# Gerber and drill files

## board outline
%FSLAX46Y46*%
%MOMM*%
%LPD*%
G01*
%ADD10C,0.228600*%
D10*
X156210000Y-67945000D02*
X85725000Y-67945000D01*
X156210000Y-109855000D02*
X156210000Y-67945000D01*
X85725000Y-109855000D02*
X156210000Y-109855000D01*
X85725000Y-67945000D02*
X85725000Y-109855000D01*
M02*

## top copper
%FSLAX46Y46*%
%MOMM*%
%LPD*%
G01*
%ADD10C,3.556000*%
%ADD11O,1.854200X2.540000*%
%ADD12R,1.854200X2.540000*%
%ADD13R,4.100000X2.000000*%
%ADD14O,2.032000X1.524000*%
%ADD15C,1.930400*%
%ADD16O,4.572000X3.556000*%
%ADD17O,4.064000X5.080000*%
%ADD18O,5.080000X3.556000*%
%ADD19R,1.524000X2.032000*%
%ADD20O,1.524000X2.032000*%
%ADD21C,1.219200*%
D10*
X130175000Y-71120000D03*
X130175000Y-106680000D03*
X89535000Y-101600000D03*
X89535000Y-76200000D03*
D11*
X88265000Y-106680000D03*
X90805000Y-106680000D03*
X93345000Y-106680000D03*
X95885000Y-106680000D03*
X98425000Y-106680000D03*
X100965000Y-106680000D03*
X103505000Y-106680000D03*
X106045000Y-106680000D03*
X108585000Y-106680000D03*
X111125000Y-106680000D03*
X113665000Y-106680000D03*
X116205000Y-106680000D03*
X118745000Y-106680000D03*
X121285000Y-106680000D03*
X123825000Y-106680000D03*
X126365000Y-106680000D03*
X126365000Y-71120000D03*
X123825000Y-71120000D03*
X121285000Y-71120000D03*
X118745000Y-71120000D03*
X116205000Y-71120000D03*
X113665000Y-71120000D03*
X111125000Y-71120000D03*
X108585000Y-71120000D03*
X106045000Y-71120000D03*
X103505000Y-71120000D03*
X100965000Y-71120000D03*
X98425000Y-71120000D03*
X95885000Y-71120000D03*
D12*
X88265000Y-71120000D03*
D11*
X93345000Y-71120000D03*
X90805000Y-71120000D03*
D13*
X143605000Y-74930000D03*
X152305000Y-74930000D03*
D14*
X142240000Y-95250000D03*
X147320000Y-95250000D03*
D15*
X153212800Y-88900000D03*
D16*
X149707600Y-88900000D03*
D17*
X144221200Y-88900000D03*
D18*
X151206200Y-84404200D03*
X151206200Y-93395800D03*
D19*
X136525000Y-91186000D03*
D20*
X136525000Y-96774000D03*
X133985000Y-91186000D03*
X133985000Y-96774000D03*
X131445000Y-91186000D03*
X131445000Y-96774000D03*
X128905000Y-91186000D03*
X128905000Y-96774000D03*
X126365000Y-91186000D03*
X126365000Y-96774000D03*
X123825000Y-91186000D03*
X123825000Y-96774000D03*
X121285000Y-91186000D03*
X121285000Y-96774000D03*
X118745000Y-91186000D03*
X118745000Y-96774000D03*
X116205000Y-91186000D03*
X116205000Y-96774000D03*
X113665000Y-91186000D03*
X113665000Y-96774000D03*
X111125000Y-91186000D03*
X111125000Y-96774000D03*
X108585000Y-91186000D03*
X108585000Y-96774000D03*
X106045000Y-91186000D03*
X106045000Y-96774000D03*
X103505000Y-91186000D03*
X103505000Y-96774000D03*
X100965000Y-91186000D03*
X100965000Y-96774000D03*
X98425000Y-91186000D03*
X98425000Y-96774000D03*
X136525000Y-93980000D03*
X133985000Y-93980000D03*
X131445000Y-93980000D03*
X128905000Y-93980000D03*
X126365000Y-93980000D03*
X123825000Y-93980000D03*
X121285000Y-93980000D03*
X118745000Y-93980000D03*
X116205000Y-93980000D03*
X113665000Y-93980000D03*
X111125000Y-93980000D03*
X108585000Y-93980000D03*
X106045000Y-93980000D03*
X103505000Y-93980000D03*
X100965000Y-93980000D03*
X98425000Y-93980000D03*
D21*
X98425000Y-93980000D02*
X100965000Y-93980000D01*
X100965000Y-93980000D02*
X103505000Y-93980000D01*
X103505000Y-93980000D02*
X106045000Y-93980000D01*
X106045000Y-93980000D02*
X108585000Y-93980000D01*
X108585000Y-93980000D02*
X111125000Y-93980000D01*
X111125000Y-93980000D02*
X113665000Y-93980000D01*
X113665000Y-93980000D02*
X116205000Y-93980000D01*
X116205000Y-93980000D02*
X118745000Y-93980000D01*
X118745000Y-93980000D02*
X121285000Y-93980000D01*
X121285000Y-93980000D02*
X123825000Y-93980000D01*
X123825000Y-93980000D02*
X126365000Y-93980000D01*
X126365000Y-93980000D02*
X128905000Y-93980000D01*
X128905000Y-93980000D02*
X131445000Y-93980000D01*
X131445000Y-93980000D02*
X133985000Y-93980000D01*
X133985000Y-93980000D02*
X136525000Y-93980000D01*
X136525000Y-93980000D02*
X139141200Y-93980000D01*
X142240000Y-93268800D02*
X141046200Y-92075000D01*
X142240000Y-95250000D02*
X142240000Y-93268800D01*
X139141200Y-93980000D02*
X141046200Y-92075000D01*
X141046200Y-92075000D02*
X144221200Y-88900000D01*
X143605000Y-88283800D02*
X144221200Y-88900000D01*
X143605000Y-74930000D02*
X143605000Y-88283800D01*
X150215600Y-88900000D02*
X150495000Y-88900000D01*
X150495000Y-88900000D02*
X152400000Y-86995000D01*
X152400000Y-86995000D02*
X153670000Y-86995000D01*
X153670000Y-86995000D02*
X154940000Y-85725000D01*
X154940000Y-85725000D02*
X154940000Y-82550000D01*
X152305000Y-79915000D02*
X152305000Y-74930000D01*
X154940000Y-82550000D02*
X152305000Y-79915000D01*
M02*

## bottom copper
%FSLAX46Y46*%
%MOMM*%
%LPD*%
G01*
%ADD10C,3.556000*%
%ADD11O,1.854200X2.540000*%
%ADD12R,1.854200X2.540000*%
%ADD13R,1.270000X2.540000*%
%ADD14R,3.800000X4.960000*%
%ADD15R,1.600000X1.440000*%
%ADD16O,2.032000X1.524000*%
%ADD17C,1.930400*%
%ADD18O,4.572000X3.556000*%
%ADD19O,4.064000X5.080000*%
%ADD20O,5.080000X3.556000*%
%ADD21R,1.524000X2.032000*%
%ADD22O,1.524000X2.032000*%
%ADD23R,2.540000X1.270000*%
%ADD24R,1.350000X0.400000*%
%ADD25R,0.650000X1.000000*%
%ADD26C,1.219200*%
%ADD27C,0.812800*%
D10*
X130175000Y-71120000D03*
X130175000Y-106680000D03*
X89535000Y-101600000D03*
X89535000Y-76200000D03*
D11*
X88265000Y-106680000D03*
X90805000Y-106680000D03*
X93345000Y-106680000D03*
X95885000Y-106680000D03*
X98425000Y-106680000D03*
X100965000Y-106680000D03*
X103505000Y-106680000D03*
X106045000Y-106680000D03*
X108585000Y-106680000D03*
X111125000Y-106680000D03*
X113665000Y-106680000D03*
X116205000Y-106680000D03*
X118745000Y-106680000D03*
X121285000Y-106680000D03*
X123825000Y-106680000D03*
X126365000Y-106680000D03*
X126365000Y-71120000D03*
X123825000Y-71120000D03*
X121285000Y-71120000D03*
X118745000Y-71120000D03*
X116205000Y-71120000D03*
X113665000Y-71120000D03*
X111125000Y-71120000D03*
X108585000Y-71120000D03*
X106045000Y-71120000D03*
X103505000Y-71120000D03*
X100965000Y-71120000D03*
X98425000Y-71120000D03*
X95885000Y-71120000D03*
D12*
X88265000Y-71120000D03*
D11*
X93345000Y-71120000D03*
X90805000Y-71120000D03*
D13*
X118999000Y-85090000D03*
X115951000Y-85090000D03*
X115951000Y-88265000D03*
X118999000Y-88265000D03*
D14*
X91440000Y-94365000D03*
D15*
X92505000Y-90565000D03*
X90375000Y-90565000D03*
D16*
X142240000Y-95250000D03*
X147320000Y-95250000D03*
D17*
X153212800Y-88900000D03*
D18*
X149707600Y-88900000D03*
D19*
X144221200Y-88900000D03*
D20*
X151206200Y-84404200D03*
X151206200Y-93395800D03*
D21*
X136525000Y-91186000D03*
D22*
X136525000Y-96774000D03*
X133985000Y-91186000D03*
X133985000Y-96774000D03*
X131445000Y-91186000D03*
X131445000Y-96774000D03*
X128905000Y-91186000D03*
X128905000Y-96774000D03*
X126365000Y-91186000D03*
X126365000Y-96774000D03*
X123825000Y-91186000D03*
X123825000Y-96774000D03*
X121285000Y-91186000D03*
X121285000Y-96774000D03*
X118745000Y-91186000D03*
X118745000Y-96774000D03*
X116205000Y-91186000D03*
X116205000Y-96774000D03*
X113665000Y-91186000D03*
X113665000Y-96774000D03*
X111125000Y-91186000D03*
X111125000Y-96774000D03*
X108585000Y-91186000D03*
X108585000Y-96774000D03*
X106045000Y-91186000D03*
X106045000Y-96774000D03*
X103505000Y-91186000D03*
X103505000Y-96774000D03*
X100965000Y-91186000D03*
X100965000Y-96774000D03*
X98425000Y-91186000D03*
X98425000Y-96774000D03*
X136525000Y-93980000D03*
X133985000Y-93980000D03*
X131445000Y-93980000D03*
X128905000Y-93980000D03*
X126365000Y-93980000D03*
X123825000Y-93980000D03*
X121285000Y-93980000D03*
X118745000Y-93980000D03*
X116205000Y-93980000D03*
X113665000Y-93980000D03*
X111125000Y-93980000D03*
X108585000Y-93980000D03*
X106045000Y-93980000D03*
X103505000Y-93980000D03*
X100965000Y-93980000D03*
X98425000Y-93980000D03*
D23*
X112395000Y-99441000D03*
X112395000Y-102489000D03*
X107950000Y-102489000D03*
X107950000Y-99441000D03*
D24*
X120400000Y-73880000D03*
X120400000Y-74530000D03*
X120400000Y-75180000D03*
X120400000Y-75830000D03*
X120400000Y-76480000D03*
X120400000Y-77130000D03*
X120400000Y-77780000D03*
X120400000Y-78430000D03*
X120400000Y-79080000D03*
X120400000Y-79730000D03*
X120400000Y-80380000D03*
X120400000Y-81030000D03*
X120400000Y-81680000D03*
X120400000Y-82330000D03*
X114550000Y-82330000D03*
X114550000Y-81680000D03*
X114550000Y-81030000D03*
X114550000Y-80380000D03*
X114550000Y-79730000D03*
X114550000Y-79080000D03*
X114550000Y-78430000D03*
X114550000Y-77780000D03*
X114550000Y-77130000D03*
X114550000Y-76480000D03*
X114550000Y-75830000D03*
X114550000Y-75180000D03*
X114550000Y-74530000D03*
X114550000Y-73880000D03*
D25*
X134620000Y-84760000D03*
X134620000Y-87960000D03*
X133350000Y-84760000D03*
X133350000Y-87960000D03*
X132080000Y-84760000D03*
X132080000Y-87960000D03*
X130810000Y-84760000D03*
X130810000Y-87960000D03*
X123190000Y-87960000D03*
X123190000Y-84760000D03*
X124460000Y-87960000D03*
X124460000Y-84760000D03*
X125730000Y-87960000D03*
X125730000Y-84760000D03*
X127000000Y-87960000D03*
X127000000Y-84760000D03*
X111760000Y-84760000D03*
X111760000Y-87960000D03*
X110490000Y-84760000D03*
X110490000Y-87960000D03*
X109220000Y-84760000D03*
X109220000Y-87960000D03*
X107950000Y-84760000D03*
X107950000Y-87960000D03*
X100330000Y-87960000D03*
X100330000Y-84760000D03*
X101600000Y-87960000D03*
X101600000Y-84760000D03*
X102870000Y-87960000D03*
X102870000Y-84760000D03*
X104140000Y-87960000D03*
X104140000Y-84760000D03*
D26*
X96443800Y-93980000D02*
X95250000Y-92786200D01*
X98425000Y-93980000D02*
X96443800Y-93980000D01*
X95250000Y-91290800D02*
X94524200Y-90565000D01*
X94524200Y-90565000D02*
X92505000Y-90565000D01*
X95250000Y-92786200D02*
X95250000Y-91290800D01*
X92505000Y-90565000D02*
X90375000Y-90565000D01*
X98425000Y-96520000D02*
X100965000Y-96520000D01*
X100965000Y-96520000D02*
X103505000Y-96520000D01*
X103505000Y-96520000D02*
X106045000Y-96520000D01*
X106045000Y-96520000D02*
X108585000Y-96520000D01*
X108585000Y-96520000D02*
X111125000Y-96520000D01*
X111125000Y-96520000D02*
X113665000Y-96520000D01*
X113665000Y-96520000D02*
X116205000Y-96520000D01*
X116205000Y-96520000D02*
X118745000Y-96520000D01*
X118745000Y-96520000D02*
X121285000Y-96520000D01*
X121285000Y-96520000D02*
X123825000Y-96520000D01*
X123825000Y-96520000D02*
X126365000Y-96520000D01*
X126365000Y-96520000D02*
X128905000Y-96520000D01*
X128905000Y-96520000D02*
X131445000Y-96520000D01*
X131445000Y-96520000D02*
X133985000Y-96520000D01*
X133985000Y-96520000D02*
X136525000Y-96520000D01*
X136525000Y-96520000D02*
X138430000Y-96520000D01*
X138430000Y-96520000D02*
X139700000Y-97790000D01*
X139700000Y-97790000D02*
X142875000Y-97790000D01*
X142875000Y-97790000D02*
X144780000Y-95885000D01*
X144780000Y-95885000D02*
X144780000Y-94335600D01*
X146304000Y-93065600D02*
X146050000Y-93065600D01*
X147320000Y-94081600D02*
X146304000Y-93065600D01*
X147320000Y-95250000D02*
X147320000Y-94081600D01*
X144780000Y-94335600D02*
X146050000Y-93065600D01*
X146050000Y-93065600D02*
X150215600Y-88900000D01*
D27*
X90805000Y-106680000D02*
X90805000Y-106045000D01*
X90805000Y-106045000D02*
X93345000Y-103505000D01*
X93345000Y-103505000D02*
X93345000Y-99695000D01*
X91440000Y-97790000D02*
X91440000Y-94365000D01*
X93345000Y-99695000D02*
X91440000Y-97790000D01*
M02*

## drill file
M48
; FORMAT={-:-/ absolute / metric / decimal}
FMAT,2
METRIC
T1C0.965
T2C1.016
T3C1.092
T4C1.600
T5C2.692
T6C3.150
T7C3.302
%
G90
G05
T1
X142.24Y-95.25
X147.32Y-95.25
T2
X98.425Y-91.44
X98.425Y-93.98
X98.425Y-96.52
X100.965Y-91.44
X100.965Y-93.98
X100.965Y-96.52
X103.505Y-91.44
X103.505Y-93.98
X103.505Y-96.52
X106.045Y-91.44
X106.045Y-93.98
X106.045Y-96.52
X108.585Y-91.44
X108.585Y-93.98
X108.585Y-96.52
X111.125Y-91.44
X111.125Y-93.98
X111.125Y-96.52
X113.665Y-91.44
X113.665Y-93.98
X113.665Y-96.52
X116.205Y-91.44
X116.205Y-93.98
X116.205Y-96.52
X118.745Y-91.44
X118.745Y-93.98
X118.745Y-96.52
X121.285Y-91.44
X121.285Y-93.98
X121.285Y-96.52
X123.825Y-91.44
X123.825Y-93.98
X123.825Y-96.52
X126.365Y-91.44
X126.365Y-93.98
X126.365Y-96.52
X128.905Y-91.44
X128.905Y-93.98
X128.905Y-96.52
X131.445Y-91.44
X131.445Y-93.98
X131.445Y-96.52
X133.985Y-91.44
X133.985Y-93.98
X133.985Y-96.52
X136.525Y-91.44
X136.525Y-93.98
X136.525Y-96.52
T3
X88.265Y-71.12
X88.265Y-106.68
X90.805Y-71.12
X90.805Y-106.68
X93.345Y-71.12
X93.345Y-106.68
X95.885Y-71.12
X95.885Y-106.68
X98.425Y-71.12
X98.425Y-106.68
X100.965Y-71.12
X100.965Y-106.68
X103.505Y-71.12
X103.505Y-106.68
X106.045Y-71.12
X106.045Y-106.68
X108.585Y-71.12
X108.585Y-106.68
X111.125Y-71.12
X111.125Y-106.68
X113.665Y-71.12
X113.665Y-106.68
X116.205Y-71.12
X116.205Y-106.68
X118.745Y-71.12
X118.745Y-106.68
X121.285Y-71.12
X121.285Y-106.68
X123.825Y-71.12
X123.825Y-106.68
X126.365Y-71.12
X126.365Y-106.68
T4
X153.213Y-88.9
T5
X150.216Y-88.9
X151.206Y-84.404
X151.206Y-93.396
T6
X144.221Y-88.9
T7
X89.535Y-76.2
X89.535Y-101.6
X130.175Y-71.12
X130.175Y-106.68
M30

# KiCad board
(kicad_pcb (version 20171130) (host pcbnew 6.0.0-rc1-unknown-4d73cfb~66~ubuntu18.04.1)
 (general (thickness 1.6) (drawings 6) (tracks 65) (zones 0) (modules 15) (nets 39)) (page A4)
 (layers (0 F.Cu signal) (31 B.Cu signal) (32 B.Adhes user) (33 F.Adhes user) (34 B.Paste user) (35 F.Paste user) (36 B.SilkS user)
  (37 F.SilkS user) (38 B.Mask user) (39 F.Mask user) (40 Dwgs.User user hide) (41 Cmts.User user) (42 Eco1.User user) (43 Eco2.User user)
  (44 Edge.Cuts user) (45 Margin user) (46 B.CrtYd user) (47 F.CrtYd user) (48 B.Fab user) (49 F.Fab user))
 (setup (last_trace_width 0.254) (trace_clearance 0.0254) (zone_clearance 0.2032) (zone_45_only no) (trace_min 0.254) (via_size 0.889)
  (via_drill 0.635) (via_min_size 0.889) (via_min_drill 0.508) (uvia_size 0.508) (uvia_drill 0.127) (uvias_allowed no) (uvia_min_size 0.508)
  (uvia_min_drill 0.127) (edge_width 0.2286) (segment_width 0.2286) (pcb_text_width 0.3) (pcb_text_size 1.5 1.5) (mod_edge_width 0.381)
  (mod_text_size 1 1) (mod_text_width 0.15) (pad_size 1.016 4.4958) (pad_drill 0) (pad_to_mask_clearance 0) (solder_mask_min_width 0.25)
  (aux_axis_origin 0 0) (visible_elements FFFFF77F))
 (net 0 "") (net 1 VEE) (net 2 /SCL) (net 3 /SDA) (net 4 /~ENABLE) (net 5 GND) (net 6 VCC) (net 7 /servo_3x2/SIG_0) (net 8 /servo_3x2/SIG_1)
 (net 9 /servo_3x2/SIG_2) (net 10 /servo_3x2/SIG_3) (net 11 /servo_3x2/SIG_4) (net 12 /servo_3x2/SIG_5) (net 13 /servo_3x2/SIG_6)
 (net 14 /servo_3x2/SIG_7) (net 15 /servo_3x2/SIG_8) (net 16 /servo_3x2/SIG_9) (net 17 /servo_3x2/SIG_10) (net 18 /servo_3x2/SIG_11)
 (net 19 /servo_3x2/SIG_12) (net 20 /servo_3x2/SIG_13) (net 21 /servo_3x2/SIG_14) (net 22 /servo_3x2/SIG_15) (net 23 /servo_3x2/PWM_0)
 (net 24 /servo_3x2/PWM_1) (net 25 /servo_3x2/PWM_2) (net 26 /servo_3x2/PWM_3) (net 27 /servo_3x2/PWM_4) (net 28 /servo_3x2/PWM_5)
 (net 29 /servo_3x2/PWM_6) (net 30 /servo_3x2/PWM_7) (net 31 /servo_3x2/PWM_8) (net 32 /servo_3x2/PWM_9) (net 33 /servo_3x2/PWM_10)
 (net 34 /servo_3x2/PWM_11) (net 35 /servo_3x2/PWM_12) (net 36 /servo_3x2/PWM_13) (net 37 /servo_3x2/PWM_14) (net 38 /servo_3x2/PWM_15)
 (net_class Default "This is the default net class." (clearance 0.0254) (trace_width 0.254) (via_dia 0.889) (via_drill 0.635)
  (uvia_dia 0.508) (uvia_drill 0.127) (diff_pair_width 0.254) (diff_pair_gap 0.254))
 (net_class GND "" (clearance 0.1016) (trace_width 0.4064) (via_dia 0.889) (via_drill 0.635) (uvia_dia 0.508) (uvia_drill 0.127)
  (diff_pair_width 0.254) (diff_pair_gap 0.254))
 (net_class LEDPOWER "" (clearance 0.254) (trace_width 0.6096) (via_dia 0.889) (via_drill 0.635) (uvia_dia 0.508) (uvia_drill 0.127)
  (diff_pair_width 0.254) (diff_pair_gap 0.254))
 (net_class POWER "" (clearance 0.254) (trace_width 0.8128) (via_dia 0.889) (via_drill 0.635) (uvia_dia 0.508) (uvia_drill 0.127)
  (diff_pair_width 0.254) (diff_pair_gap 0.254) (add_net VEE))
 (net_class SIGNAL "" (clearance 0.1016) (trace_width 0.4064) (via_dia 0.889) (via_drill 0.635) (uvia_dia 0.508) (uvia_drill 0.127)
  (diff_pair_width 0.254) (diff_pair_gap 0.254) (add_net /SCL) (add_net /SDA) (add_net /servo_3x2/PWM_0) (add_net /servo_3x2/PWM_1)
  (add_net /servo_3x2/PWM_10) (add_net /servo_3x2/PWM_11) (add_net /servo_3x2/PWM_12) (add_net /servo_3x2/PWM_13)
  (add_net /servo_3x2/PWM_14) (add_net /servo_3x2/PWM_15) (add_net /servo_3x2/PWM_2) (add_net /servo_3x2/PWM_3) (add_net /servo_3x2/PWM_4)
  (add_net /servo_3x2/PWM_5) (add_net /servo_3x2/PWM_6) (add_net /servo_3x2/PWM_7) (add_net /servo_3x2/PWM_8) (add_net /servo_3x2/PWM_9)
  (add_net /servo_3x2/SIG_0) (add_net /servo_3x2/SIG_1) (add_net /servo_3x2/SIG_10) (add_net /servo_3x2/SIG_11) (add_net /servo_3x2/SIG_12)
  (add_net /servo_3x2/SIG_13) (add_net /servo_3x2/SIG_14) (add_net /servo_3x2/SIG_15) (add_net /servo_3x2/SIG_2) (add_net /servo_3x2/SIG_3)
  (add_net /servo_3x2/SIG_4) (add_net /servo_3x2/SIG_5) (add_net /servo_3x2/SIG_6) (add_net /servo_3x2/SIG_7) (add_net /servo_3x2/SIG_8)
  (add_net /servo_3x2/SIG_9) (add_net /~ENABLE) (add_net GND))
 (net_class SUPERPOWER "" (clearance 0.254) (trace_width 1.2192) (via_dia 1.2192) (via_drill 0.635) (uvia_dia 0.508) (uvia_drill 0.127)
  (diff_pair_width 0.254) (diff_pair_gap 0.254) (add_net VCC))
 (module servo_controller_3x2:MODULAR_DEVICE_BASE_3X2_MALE (layer F.Cu) (at 107.315 88.9)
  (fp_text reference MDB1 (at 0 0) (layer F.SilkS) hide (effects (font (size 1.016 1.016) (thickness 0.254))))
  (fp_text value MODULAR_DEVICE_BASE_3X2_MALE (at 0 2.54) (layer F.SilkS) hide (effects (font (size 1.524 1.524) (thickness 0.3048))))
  (pad "" thru_hole circle (at 22.86 -17.78) (size 3.556 3.556) (drill 3.302) (layers *.Cu *.Mask F.SilkS))
  (pad "" thru_hole circle (at 22.86 17.78) (size 3.556 3.556) (drill 3.302) (layers *.Cu *.Mask F.SilkS))
  (pad "" thru_hole circle (at -17.78 12.7) (size 3.556 3.556) (drill 3.302) (layers *.Cu *.Mask F.SilkS))
  (pad "" thru_hole circle (at -17.78 -12.7) (size 3.556 3.556) (drill 3.302) (layers *.Cu *.Mask F.SilkS))
  (pad AREF thru_hole oval (at -19.05 17.78) (size 1.8542 2.54) (drill 1.0922) (layers *.Cu *.Mask))
  (pad VEE thru_hole oval (at -16.51 17.78) (size 1.8542 2.54) (drill 1.0922) (layers *.Cu *.Mask) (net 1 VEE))
  (pad AGND thru_hole oval (at -13.97 17.78) (size 1.8542 2.54) (drill 1.0922) (layers *.Cu *.Mask))
  (pad 3V3 thru_hole oval (at -11.43 17.78) (size 1.8542 2.54) (drill 1.0922) (layers *.Cu *.Mask))
  (pad 23 thru_hole oval (at -8.89 17.78) (size 1.8542 2.54) (drill 1.0922) (layers *.Cu *.Mask))
  (pad 22 thru_hole oval (at -6.35 17.78) (size 1.8542 2.54) (drill 1.0922) (layers *.Cu *.Mask))
  (pad 21 thru_hole oval (at -3.81 17.78) (size 1.8542 2.54) (drill 1.0922) (layers *.Cu *.Mask))
  (pad 20 thru_hole oval (at -1.27 17.78) (size 1.8542 2.54) (drill 1.0922) (layers *.Cu *.Mask))
  (pad 19 thru_hole oval (at 1.27 17.78) (size 1.8542 2.54) (drill 1.0922) (layers *.Cu *.Mask) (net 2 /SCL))
  (pad 18 thru_hole oval (at 3.81 17.78) (size 1.8542 2.54) (drill 1.0922) (layers *.Cu *.Mask) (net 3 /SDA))
  (pad 17 thru_hole oval (at 6.35 17.78) (size 1.8542 2.54) (drill 1.0922) (layers *.Cu *.Mask))
  (pad 16 thru_hole oval (at 8.89 17.78) (size 1.8542 2.54) (drill 1.0922) (layers *.Cu *.Mask))
  (pad 15 thru_hole oval (at 11.43 17.78) (size 1.8542 2.54) (drill 1.0922) (layers *.Cu *.Mask))
  (pad 14 thru_hole oval (at 13.97 17.78) (size 1.8542 2.54) (drill 1.0922) (layers *.Cu *.Mask))
  (pad 13 thru_hole oval (at 16.51 17.78) (size 1.8542 2.54) (drill 1.0922) (layers *.Cu *.Mask))
  (pad DAC thru_hole oval (at 19.05 17.78) (size 1.8542 2.54) (drill 1.0922) (layers *.Cu *.Mask))
  (pad 28 thru_hole oval (at 19.05 -17.78) (size 1.8542 2.54) (drill 1.0922) (layers *.Cu *.Mask))
  (pad 12 thru_hole oval (at 16.51 -17.78) (size 1.8542 2.54) (drill 1.0922) (layers *.Cu *.Mask))
  (pad 11 thru_hole oval (at 13.97 -17.78) (size 1.8542 2.54) (drill 1.0922) (layers *.Cu *.Mask))
  (pad 10 thru_hole oval (at 11.43 -17.78) (size 1.8542 2.54) (drill 1.0922) (layers *.Cu *.Mask))
  (pad 9 thru_hole oval (at 8.89 -17.78) (size 1.8542 2.54) (drill 1.0922) (layers *.Cu *.Mask))
  (pad 29 thru_hole oval (at 6.35 -17.78) (size 1.8542 2.54) (drill 1.0922) (layers *.Cu *.Mask))
  (pad 30 thru_hole oval (at 3.81 -17.78) (size 1.8542 2.54) (drill 1.0922) (layers *.Cu *.Mask))
  (pad 6 thru_hole oval (at 1.27 -17.78) (size 1.8542 2.54) (drill 1.0922) (layers *.Cu *.Mask))
  (pad 5 thru_hole oval (at -1.27 -17.78) (size 1.8542 2.54) (drill 1.0922) (layers *.Cu *.Mask))
  (pad 4 thru_hole oval (at -3.81 -17.78) (size 1.8542 2.54) (drill 1.0922) (layers *.Cu *.Mask))
  (pad 3 thru_hole oval (at -6.35 -17.78) (size 1.8542 2.54) (drill 1.0922) (layers *.Cu *.Mask))
  (pad 2 thru_hole oval (at -8.89 -17.78) (size 1.8542 2.54) (drill 1.0922) (layers *.Cu *.Mask) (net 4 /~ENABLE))
  (pad 25 thru_hole oval (at -11.43 -17.78) (size 1.8542 2.54) (drill 1.0922) (layers *.Cu *.Mask))
  (pad VDD thru_hole rect (at -19.05 -17.78) (size 1.8542 2.54) (drill 1.0922) (layers *.Cu *.Mask))
  (pad 24 thru_hole oval (at -13.97 -17.78) (size 1.8542 2.54) (drill 1.0922) (layers *.Cu *.Mask))
  (pad GND thru_hole oval (at -16.51 -17.78) (size 1.8542 2.54) (drill 1.0922) (layers *.Cu *.Mask) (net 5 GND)))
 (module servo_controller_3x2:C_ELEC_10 (layer F.Cu) (at 147.955 74.93 180)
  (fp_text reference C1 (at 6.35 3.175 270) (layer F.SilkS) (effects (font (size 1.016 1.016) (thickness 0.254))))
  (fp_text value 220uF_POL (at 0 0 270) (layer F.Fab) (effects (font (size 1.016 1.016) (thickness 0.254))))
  (pad 1 smd rect (at 4.35 0 180) (size 4.1 2) (layers F.Cu F.Paste F.Mask) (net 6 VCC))
  (pad 2 smd rect (at -4.35 0 180) (size 4.1 2) (layers F.Cu F.Paste F.Mask) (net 5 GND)))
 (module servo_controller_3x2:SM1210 (layer B.Cu) (at 117.475 85.09)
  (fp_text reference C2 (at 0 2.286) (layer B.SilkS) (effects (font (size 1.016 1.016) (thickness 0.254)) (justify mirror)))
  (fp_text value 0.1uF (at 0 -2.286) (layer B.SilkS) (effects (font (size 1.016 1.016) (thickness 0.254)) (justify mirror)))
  (pad 2 smd rect (at 1.524 0) (size 1.27 2.54) (layers B.Cu B.Paste B.Mask) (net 5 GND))
  (pad 1 smd rect (at -1.524 0) (size 1.27 2.54) (layers B.Cu B.Paste B.Mask) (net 1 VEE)))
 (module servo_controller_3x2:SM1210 (layer B.Cu) (at 117.475 88.265)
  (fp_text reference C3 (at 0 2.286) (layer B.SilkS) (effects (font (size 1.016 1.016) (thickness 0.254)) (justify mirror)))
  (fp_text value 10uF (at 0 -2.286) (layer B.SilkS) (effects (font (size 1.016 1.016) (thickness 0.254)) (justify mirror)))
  (pad 1 smd rect (at -1.524 0) (size 1.27 2.54) (layers B.Cu B.Paste B.Mask) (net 1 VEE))
  (pad 2 smd rect (at 1.524 0) (size 1.27 2.54) (layers B.Cu B.Paste B.Mask) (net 5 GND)))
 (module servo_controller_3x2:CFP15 (layer B.Cu) (at 91.44 93.345 180)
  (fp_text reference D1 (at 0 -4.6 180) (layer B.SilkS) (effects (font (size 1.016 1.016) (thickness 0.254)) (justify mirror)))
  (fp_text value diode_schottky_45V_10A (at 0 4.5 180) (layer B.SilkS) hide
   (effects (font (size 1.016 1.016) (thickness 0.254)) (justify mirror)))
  (pad 1 smd rect (at 0 -1.02 180) (size 3.8 4.96) (layers B.Cu B.Paste B.Mask) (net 1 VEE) (solder_mask_margin 0.1) (clearance 0.1))
  (pad 2 smd rect (at -1.065 2.78 180) (size 1.6 1.44) (layers B.Cu B.Paste B.Mask) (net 6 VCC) (solder_mask_margin 0.1) (clearance 0.1))
  (pad 2 smd rect (at 1.065 2.78 180) (size 1.6 1.44) (layers B.Cu B.Paste B.Mask) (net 6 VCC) (solder_mask_margin 0.1) (clearance 0.1)))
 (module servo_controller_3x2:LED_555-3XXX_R (layer F.Cu) (at 144.78 95.25 90)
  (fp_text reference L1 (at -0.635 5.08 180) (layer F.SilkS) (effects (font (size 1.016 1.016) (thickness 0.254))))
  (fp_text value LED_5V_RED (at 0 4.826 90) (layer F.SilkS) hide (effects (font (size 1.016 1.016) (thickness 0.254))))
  (pad 1 thru_hole oval (at 0 -2.54 90) (size 1.524 2.032) (drill 0.9652) (layers *.Cu *.Mask) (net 6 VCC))
  (pad 2 thru_hole oval (at 0 2.54 90) (size 1.524 2.032) (drill 0.9652) (layers *.Cu *.Mask) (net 5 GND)))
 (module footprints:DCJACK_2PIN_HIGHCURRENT (layer F.Cu) (at 156.21 88.9 270)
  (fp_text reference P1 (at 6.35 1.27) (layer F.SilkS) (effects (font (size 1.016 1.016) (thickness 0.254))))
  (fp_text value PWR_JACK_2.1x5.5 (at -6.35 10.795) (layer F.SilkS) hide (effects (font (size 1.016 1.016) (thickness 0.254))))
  (pad "" thru_hole circle (at 0 2.9972 270) (size 1.9304 1.9304) (drill 1.6002) (layers *.Cu *.Mask))
  (pad 2 thru_hole oval (at 0 5.9944 270) (size 3.556 4.572) (drill 2.6924 (offset 0 0.508)) (layers *.Cu *.Mask) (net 5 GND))
  (pad 1 thru_hole oval (at 0 11.9888 270) (size 5.08 4.064) (drill 3.1496) (layers *.Cu *.Mask) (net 6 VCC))
  (pad "" thru_hole oval (at -4.4958 5.0038 270) (size 3.556 5.08) (drill 2.6924) (layers *.Cu *.Mask))
  (pad "" thru_hole oval (at 4.4958 5.0038 270) (size 3.556 5.08) (drill 2.6924) (layers *.Cu *.Mask)))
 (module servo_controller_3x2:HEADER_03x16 (layer F.Cu) (at 117.475 93.98)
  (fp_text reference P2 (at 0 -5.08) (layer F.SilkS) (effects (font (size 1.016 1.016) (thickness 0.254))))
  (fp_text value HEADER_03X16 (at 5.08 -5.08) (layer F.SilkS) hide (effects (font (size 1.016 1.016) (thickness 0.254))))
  (pad 1 thru_hole rect (at 19.05 -2.54) (size 1.524 2.032) (drill 1.016 (offset 0 -0.254)) (layers *.Cu *.Mask) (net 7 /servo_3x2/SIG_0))
  (pad 3 thru_hole oval (at 19.05 2.54) (size 1.524 2.032) (drill 1.016 (offset 0 0.254)) (layers *.Cu *.Mask) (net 5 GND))
  (pad 4 thru_hole oval (at 16.51 -2.54) (size 1.524 2.032) (drill 1.016 (offset 0 -0.254)) (layers *.Cu *.Mask) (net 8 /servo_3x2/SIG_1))
  (pad 6 thru_hole oval (at 16.51 2.54) (size 1.524 2.032) (drill 1.016 (offset 0 0.254)) (layers *.Cu *.Mask) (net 5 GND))
  (pad 7 thru_hole oval (at 13.97 -2.54) (size 1.524 2.032) (drill 1.016 (offset 0 -0.254)) (layers *.Cu *.Mask) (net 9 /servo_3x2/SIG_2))
  (pad 9 thru_hole oval (at 13.97 2.54) (size 1.524 2.032) (drill 1.016 (offset 0 0.254)) (layers *.Cu *.Mask) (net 5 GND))
  (pad 10 thru_hole oval (at 11.43 -2.54) (size 1.524 2.032) (drill 1.016 (offset 0 -0.254)) (layers *.Cu *.Mask) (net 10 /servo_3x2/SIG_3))
  (pad 12 thru_hole oval (at 11.43 2.54) (size 1.524 2.032) (drill 1.016 (offset 0 0.254)) (layers *.Cu *.Mask) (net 5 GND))
  (pad 13 thru_hole oval (at 8.89 -2.54) (size 1.524 2.032) (drill 1.016 (offset 0 -0.254)) (layers *.Cu *.Mask) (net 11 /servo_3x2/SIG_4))
  (pad 15 thru_hole oval (at 8.89 2.54) (size 1.524 2.032) (drill 1.016 (offset 0 0.254)) (layers *.Cu *.Mask) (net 5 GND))
  (pad 16 thru_hole oval (at 6.35 -2.54) (size 1.524 2.032) (drill 1.016 (offset 0 -0.254)) (layers *.Cu *.Mask) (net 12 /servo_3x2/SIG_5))
  (pad 18 thru_hole oval (at 6.35 2.54) (size 1.524 2.032) (drill 1.016 (offset 0 0.254)) (layers *.Cu *.Mask) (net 5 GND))
  (pad 19 thru_hole oval (at 3.81 -2.54) (size 1.524 2.032) (drill 1.016 (offset 0 -0.254)) (layers *.Cu *.Mask) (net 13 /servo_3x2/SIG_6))
  (pad 21 thru_hole oval (at 3.81 2.54) (size 1.524 2.032) (drill 1.016 (offset 0 0.254)) (layers *.Cu *.Mask) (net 5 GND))
  (pad 22 thru_hole oval (at 1.27 -2.54) (size 1.524 2.032) (drill 1.016 (offset 0 -0.254)) (layers *.Cu *.Mask) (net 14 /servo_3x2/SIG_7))
  (pad 24 thru_hole oval (at 1.27 2.54) (size 1.524 2.032) (drill 1.016 (offset 0 0.254)) (layers *.Cu *.Mask) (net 5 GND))
  (pad 25 thru_hole oval (at -1.27 -2.54) (size 1.524 2.032) (drill 1.016 (offset 0 -0.254)) (layers *.Cu *.Mask) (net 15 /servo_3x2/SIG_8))
  (pad 27 thru_hole oval (at -1.27 2.54) (size 1.524 2.032) (drill 1.016 (offset 0 0.254)) (layers *.Cu *.Mask) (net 5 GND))
  (pad 28 thru_hole oval (at -3.81 -2.54) (size 1.524 2.032) (drill 1.016 (offset 0 -0.254)) (layers *.Cu *.Mask) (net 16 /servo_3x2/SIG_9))
  (pad 30 thru_hole oval (at -3.81 2.54) (size 1.524 2.032) (drill 1.016 (offset 0 0.254)) (layers *.Cu *.Mask) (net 5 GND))
  (pad 31 thru_hole oval (at -6.35 -2.54) (size 1.524 2.032) (drill 1.016 (offset 0 -0.254)) (layers *.Cu *.Mask) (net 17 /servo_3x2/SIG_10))
  (pad 33 thru_hole oval (at -6.35 2.54) (size 1.524 2.032) (drill 1.016 (offset 0 0.254)) (layers *.Cu *.Mask) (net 5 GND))
  (pad 34 thru_hole oval (at -8.89 -2.54) (size 1.524 2.032) (drill 1.016 (offset 0 -0.254)) (layers *.Cu *.Mask) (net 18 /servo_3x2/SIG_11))
  (pad 36 thru_hole oval (at -8.89 2.54) (size 1.524 2.032) (drill 1.016 (offset 0 0.254)) (layers *.Cu *.Mask) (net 5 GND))
  (pad 37 thru_hole oval (at -11.43 -2.54) (size 1.524 2.032) (drill 1.016 (offset 0 -0.254)) (layers *.Cu *.Mask)
   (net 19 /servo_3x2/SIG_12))
  (pad 39 thru_hole oval (at -11.43 2.54) (size 1.524 2.032) (drill 1.016 (offset 0 0.254)) (layers *.Cu *.Mask) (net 5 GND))
  (pad 40 thru_hole oval (at -13.97 -2.54) (size 1.524 2.032) (drill 1.016 (offset 0 -0.254)) (layers *.Cu *.Mask)
   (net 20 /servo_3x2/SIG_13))
  (pad 42 thru_hole oval (at -13.97 2.54) (size 1.524 2.032) (drill 1.016 (offset 0 0.254)) (layers *.Cu *.Mask) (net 5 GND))
  (pad 43 thru_hole oval (at -16.51 -2.54) (size 1.524 2.032) (drill 1.016 (offset 0 -0.254)) (layers *.Cu *.Mask)
   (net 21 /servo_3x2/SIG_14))
  (pad 45 thru_hole oval (at -16.51 2.54) (size 1.524 2.032) (drill 1.016 (offset 0 0.254)) (layers *.Cu *.Mask) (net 5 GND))
  (pad 46 thru_hole oval (at -19.05 -2.54) (size 1.524 2.032) (drill 1.016 (offset 0 -0.254)) (layers *.Cu *.Mask)
   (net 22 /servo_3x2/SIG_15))
  (pad 48 thru_hole oval (at -19.05 2.54) (size 1.524 2.032) (drill 1.016 (offset 0 0.254)) (layers *.Cu *.Mask) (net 5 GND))
  (pad 2 thru_hole oval (at 19.05 0) (size 1.524 2.032) (drill 1.016) (layers *.Cu *.Mask) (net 6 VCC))
  (pad 5 thru_hole oval (at 16.51 0) (size 1.524 2.032) (drill 1.016) (layers *.Cu *.Mask) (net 6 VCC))
  (pad 8 thru_hole oval (at 13.97 0) (size 1.524 2.032) (drill 1.016) (layers *.Cu *.Mask) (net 6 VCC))
  (pad 11 thru_hole oval (at 11.43 0) (size 1.524 2.032) (drill 1.016) (layers *.Cu *.Mask) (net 6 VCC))
  (pad 14 thru_hole oval (at 8.89 0) (size 1.524 2.032) (drill 1.016) (layers *.Cu *.Mask) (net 6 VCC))
  (pad 17 thru_hole oval (at 6.35 0) (size 1.524 2.032) (drill 1.016) (layers *.Cu *.Mask) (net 6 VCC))
  (pad 20 thru_hole oval (at 3.81 0) (size 1.524 2.032) (drill 1.016) (layers *.Cu *.Mask) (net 6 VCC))
  (pad 23 thru_hole oval (at 1.27 0) (size 1.524 2.032) (drill 1.016) (layers *.Cu *.Mask) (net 6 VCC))
  (pad 26 thru_hole oval (at -1.27 0) (size 1.524 2.032) (drill 1.016) (layers *.Cu *.Mask) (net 6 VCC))
  (pad 29 thru_hole oval (at -3.81 0) (size 1.524 2.032) (drill 1.016) (layers *.Cu *.Mask) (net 6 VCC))
  (pad 32 thru_hole oval (at -6.35 0) (size 1.524 2.032) (drill 1.016) (layers *.Cu *.Mask) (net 6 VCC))
  (pad 35 thru_hole oval (at -8.89 0) (size 1.524 2.032) (drill 1.016) (layers *.Cu *.Mask) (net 6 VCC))
  (pad 38 thru_hole oval (at -11.43 0) (size 1.524 2.032) (drill 1.016) (layers *.Cu *.Mask) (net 6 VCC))
  (pad 41 thru_hole oval (at -13.97 0) (size 1.524 2.032) (drill 1.016) (layers *.Cu *.Mask) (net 6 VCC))
  (pad 44 thru_hole oval (at -16.51 0) (size 1.524 2.032) (drill 1.016) (layers *.Cu *.Mask) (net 6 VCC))
  (pad 47 thru_hole oval (at -19.05 0) (size 1.524 2.032) (drill 1.016) (layers *.Cu *.Mask) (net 6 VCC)))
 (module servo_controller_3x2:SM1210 (layer B.Cu) (at 112.395 100.965 270)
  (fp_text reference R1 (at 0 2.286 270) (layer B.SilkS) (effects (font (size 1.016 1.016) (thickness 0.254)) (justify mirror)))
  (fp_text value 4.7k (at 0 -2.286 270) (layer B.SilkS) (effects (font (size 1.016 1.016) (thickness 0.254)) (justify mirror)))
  (pad 1 smd rect (at -1.524 0 270) (size 1.27 2.54) (layers B.Cu B.Paste B.Mask) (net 1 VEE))
  (pad 2 smd rect (at 1.524 0 270) (size 1.27 2.54) (layers B.Cu B.Paste B.Mask) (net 3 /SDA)))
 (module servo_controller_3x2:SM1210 (layer B.Cu) (at 107.95 100.965 270)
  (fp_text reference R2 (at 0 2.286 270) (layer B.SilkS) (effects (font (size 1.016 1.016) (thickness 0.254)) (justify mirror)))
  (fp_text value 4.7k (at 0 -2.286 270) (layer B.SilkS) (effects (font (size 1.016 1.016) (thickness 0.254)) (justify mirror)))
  (pad 2 smd rect (at 1.524 0 270) (size 1.27 2.54) (layers B.Cu B.Paste B.Mask) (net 2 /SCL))
  (pad 1 smd rect (at -1.524 0 270) (size 1.27 2.54) (layers B.Cu B.Paste B.Mask) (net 1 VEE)))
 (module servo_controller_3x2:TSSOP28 (layer B.Cu) (at 117.475 78.105 270)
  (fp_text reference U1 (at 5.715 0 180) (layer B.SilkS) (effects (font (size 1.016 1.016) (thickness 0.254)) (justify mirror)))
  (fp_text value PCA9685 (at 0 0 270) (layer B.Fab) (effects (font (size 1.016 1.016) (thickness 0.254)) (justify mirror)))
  (pad 1 smd rect (at -4.225 -2.925 270) (size 0.4 1.35) (layers B.Cu B.Paste B.Mask) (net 5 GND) (solder_mask_margin 0.075)
   (clearance 0.075))
  (pad 2 smd rect (at -3.575 -2.925 270) (size 0.4 1.35) (layers B.Cu B.Paste B.Mask) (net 5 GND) (solder_mask_margin 0.075)
   (clearance 0.075))
  (pad 3 smd rect (at -2.925 -2.925 270) (size 0.4 1.35) (layers B.Cu B.Paste B.Mask) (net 5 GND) (solder_mask_margin 0.075)
   (clearance 0.075))
  (pad 4 smd rect (at -2.275 -2.925 270) (size 0.4 1.35) (layers B.Cu B.Paste B.Mask) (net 5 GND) (solder_mask_margin 0.075)
   (clearance 0.075))
  (pad 5 smd rect (at -1.625 -2.925 270) (size 0.4 1.35) (layers B.Cu B.Paste B.Mask) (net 5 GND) (solder_mask_margin 0.075)
   (clearance 0.075))
  (pad 6 smd rect (at -0.975 -2.925 270) (size 0.4 1.35) (layers B.Cu B.Paste B.Mask) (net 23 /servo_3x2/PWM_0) (solder_mask_margin 0.075)
   (clearance 0.075))
  (pad 7 smd rect (at -0.325 -2.925 270) (size 0.4 1.35) (layers B.Cu B.Paste B.Mask) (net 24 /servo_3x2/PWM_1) (solder_mask_margin 0.075)
   (clearance 0.075))
  (pad 8 smd rect (at 0.325 -2.925 270) (size 0.4 1.35) (layers B.Cu B.Paste B.Mask) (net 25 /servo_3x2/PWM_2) (solder_mask_margin 0.075)
   (clearance 0.075))
  (pad 9 smd rect (at 0.975 -2.925 270) (size 0.4 1.35) (layers B.Cu B.Paste B.Mask) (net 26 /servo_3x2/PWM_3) (solder_mask_margin 0.075)
   (clearance 0.075))
  (pad 10 smd rect (at 1.625 -2.925 270) (size 0.4 1.35) (layers B.Cu B.Paste B.Mask) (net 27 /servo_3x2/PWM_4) (solder_mask_margin 0.075)
   (clearance 0.075))
  (pad 11 smd rect (at 2.275 -2.925 270) (size 0.4 1.35) (layers B.Cu B.Paste B.Mask) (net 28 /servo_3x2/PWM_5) (solder_mask_margin 0.075)
   (clearance 0.075))
  (pad 12 smd rect (at 2.925 -2.925 270) (size 0.4 1.35) (layers B.Cu B.Paste B.Mask) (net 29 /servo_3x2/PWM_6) (solder_mask_margin 0.075)
   (clearance 0.075))
  (pad 13 smd rect (at 3.575 -2.925 270) (size 0.4 1.35) (layers B.Cu B.Paste B.Mask) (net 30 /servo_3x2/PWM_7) (solder_mask_margin 0.075)
   (clearance 0.075))
  (pad 14 smd rect (at 4.225 -2.925 270) (size 0.4 1.35) (layers B.Cu B.Paste B.Mask) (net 5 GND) (solder_mask_margin 0.075)
   (clearance 0.075))
  (pad 15 smd rect (at 4.225 2.925 270) (size 0.4 1.35) (layers B.Cu B.Paste B.Mask) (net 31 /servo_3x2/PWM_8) (solder_mask_margin 0.075)
   (clearance 0.075))
  (pad 16 smd rect (at 3.575 2.925 270) (size 0.4 1.35) (layers B.Cu B.Paste B.Mask) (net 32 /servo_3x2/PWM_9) (solder_mask_margin 0.075)
   (clearance 0.075))
  (pad 17 smd rect (at 2.925 2.925 270) (size 0.4 1.35) (layers B.Cu B.Paste B.Mask) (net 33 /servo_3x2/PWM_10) (solder_mask_margin 0.075)
   (clearance 0.075))
  (pad 18 smd rect (at 2.275 2.925 270) (size 0.4 1.35) (layers B.Cu B.Paste B.Mask) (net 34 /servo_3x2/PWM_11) (solder_mask_margin 0.075)
   (clearance 0.075))
  (pad 19 smd rect (at 1.625 2.925 270) (size 0.4 1.35) (layers B.Cu B.Paste B.Mask) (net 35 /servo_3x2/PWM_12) (solder_mask_margin 0.075)
   (clearance 0.075))
  (pad 20 smd rect (at 0.975 2.925 270) (size 0.4 1.35) (layers B.Cu B.Paste B.Mask) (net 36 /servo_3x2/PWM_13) (solder_mask_margin 0.075)
   (clearance 0.075))
  (pad 21 smd rect (at 0.325 2.925 270) (size 0.4 1.35) (layers B.Cu B.Paste B.Mask) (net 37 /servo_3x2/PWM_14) (solder_mask_margin 0.075)
   (clearance 0.075))
  (pad 22 smd rect (at -0.325 2.925 270) (size 0.4 1.35) (layers B.Cu B.Paste B.Mask) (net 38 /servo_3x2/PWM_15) (solder_mask_margin 0.075)
   (clearance 0.075))
  (pad 23 smd rect (at -0.975 2.925 270) (size 0.4 1.35) (layers B.Cu B.Paste B.Mask) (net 4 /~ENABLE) (solder_mask_margin 0.075)
   (clearance 0.075))
  (pad 24 smd rect (at -1.625 2.925 270) (size 0.4 1.35) (layers B.Cu B.Paste B.Mask) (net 5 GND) (solder_mask_margin 0.075)
   (clearance 0.075))
  (pad 25 smd rect (at -2.275 2.925 270) (size 0.4 1.35) (layers B.Cu B.Paste B.Mask) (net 5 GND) (solder_mask_margin 0.075)
   (clearance 0.075))
  (pad 26 smd rect (at -2.925 2.925 270) (size 0.4 1.35) (layers B.Cu B.Paste B.Mask) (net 2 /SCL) (solder_mask_margin 0.075)
   (clearance 0.075))
  (pad 27 smd rect (at -3.575 2.925 270) (size 0.4 1.35) (layers B.Cu B.Paste B.Mask) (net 3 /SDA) (solder_mask_margin 0.075)
   (clearance 0.075))
  (pad 28 smd rect (at -4.225 2.925 270) (size 0.4 1.35) (layers B.Cu B.Paste B.Mask) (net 1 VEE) (solder_mask_margin 0.075)
   (clearance 0.075)))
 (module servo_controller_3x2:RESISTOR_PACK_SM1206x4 (layer B.Cu) (at 132.715 86.36 180)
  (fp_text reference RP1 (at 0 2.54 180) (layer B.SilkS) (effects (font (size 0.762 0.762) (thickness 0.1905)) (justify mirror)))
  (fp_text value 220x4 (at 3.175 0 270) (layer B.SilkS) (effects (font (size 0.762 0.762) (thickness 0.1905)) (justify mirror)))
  (pad 7 smd rect (at -1.905 1.6 180) (size 0.65 1) (layers B.Cu B.Paste B.Mask) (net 23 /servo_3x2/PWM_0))
  (pad 8 smd rect (at -1.905 -1.6 180) (size 0.65 1) (layers B.Cu B.Paste B.Mask) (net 7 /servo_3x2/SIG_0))
  (pad 5 smd rect (at -0.635 1.6 180) (size 0.65 1) (layers B.Cu B.Paste B.Mask) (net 24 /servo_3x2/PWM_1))
  (pad 6 smd rect (at -0.635 -1.6 180) (size 0.65 1) (layers B.Cu B.Paste B.Mask) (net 8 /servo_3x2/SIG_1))
  (pad 3 smd rect (at 0.635 1.6 180) (size 0.65 1) (layers B.Cu B.Paste B.Mask) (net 25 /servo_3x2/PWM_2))
  (pad 4 smd rect (at 0.635 -1.6 180) (size 0.65 1) (layers B.Cu B.Paste B.Mask) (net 9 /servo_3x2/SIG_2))
  (pad 1 smd rect (at 1.905 1.6 180) (size 0.65 1) (layers B.Cu B.Paste B.Mask) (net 26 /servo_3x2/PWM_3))
  (pad 2 smd rect (at 1.905 -1.6 180) (size 0.65 1) (layers B.Cu B.Paste B.Mask) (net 10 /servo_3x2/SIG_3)))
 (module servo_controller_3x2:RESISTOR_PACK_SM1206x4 (layer B.Cu) (at 125.095 86.36 180)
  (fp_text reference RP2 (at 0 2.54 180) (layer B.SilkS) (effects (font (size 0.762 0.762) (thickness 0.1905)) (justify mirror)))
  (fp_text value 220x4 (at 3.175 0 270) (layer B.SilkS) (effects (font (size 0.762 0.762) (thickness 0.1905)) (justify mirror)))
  (pad 2 smd rect (at 1.905 -1.6 180) (size 0.65 1) (layers B.Cu B.Paste B.Mask) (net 14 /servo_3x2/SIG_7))
  (pad 1 smd rect (at 1.905 1.6 180) (size 0.65 1) (layers B.Cu B.Paste B.Mask) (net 30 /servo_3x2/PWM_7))
  (pad 4 smd rect (at 0.635 -1.6 180) (size 0.65 1) (layers B.Cu B.Paste B.Mask) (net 13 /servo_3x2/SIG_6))
  (pad 3 smd rect (at 0.635 1.6 180) (size 0.65 1) (layers B.Cu B.Paste B.Mask) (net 29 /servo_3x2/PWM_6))
  (pad 6 smd rect (at -0.635 -1.6 180) (size 0.65 1) (layers B.Cu B.Paste B.Mask) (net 12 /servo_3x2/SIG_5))
  (pad 5 smd rect (at -0.635 1.6 180) (size 0.65 1) (layers B.Cu B.Paste B.Mask) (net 28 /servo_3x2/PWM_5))
  (pad 8 smd rect (at -1.905 -1.6 180) (size 0.65 1) (layers B.Cu B.Paste B.Mask) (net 11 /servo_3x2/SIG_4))
  (pad 7 smd rect (at -1.905 1.6 180) (size 0.65 1) (layers B.Cu B.Paste B.Mask) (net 27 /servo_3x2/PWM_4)))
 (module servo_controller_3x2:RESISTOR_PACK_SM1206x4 (layer B.Cu) (at 109.855 86.36 180)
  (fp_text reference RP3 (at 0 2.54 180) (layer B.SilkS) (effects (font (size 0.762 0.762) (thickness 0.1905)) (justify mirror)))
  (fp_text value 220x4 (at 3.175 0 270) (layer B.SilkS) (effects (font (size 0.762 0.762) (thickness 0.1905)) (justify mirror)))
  (pad 7 smd rect (at -1.905 1.6 180) (size 0.65 1) (layers B.Cu B.Paste B.Mask) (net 31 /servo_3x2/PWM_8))
  (pad 8 smd rect (at -1.905 -1.6 180) (size 0.65 1) (layers B.Cu B.Paste B.Mask) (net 15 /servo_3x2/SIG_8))
  (pad 5 smd rect (at -0.635 1.6 180) (size 0.65 1) (layers B.Cu B.Paste B.Mask) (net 32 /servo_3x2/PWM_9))
  (pad 6 smd rect (at -0.635 -1.6 180) (size 0.65 1) (layers B.Cu B.Paste B.Mask) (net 16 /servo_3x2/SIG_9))
  (pad 3 smd rect (at 0.635 1.6 180) (size 0.65 1) (layers B.Cu B.Paste B.Mask) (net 33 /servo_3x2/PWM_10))
  (pad 4 smd rect (at 0.635 -1.6 180) (size 0.65 1) (layers B.Cu B.Paste B.Mask) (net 17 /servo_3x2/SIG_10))
  (pad 1 smd rect (at 1.905 1.6 180) (size 0.65 1) (layers B.Cu B.Paste B.Mask) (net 34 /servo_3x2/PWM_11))
  (pad 2 smd rect (at 1.905 -1.6 180) (size 0.65 1) (layers B.Cu B.Paste B.Mask) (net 18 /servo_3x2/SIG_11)))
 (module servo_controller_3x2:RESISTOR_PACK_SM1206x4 (layer B.Cu) (at 102.235 86.36 180)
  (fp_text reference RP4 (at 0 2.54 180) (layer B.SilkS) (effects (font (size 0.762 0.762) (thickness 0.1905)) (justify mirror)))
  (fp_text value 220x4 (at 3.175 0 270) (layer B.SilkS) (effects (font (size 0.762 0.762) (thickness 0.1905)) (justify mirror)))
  (pad 2 smd rect (at 1.905 -1.6 180) (size 0.65 1) (layers B.Cu B.Paste B.Mask) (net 22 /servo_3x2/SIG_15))
  (pad 1 smd rect (at 1.905 1.6 180) (size 0.65 1) (layers B.Cu B.Paste B.Mask) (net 38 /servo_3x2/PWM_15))
  (pad 4 smd rect (at 0.635 -1.6 180) (size 0.65 1) (layers B.Cu B.Paste B.Mask) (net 21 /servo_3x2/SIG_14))
  (pad 3 smd rect (at 0.635 1.6 180) (size 0.65 1) (layers B.Cu B.Paste B.Mask) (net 37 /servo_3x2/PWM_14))
  (pad 6 smd rect (at -0.635 -1.6 180) (size 0.65 1) (layers B.Cu B.Paste B.Mask) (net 20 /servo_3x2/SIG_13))
  (pad 5 smd rect (at -0.635 1.6 180) (size 0.65 1) (layers B.Cu B.Paste B.Mask) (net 36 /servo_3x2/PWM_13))
  (pad 8 smd rect (at -1.905 -1.6 180) (size 0.65 1) (layers B.Cu B.Paste B.Mask) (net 19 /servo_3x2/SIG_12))
  (pad 7 smd rect (at -1.905 1.6 180) (size 0.65 1) (layers B.Cu B.Paste B.Mask) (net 35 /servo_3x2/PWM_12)))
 (gr_line (start 156.21 67.945) (end 85.725 67.945) (angle 90) (layer Edge.Cuts) (width 0.2286))
 (gr_line (start 156.21 109.855) (end 156.21 67.945) (angle 90) (layer Edge.Cuts) (width 0.2286))
 (gr_line (start 85.725 109.855) (end 156.21 109.855) (angle 90) (layer Edge.Cuts) (width 0.2286))
 (gr_line (start 85.725 67.945) (end 85.725 109.855) (angle 90) (layer Edge.Cuts) (width 0.2286))
 (segment (start 98.425 93.98) (end 100.965 93.98) (width 1.2192) (layer F.Cu) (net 6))
 (segment (start 100.965 93.98) (end 103.505 93.98) (width 1.2192) (layer F.Cu) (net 6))
 (segment (start 103.505 93.98) (end 106.045 93.98) (width 1.2192) (layer F.Cu) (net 6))
 (segment (start 106.045 93.98) (end 108.585 93.98) (width 1.2192) (layer F.Cu) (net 6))
 (segment (start 108.585 93.98) (end 111.125 93.98) (width 1.2192) (layer F.Cu) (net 6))
 (segment (start 111.125 93.98) (end 113.665 93.98) (width 1.2192) (layer F.Cu) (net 6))
 (segment (start 113.665 93.98) (end 116.205 93.98) (width 1.2192) (layer F.Cu) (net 6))
 (segment (start 116.205 93.98) (end 118.745 93.98) (width 1.2192) (layer F.Cu) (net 6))
 (segment (start 118.745 93.98) (end 121.285 93.98) (width 1.2192) (layer F.Cu) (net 6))
 (segment (start 121.285 93.98) (end 123.825 93.98) (width 1.2192) (layer F.Cu) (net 6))
 (segment (start 123.825 93.98) (end 126.365 93.98) (width 1.2192) (layer F.Cu) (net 6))
 (segment (start 126.365 93.98) (end 128.905 93.98) (width 1.2192) (layer F.Cu) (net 6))
 (segment (start 128.905 93.98) (end 131.445 93.98) (width 1.2192) (layer F.Cu) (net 6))
 (segment (start 131.445 93.98) (end 133.985 93.98) (width 1.2192) (layer F.Cu) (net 6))
 (segment (start 133.985 93.98) (end 136.525 93.98) (width 1.2192) (layer F.Cu) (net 6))
 (segment (start 136.525 93.98) (end 139.1412 93.98) (width 1.2192) (layer F.Cu) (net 6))
 (segment (start 142.24 93.2688) (end 141.0462 92.075) (width 1.2192) (layer F.Cu) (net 6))
 (segment (start 142.24 95.25) (end 142.24 93.2688) (width 1.2192) (layer F.Cu) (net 6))
 (segment (start 139.1412 93.98) (end 141.0462 92.075) (width 1.2192) (layer F.Cu) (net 6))
 (segment (start 141.0462 92.075) (end 144.2212 88.9) (width 1.2192) (layer F.Cu) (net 6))
 (segment (start 143.605 88.2838) (end 144.2212 88.9) (width 1.2192) (layer F.Cu) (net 6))
 (segment (start 143.605 74.93) (end 143.605 88.2838) (width 1.2192) (layer F.Cu) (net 6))
 (segment (start 96.4438 93.98) (end 95.25 92.7862) (width 1.2192) (layer B.Cu) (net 6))
 (segment (start 98.425 93.98) (end 96.4438 93.98) (width 1.2192) (layer B.Cu) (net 6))
 (segment (start 95.25 91.2908) (end 94.5242 90.565) (width 1.2192) (layer B.Cu) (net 6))
 (segment (start 94.5242 90.565) (end 92.505 90.565) (width 1.2192) (layer B.Cu) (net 6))
 (segment (start 95.25 92.7862) (end 95.25 91.2908) (width 1.2192) (layer B.Cu) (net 6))
 (segment (start 92.505 90.565) (end 90.375 90.565) (width 1.2192) (layer B.Cu) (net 6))
 (segment (start 150.2156 88.9) (end 150.495 88.9) (width 1.2192) (layer F.Cu) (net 5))
 (segment (start 150.495 88.9) (end 152.4 86.995) (width 1.2192) (layer F.Cu) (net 5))
 (segment (start 152.4 86.995) (end 153.67 86.995) (width 1.2192) (layer F.Cu) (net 5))
 (segment (start 153.67 86.995) (end 154.94 85.725) (width 1.2192) (layer F.Cu) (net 5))
 (segment (start 154.94 85.725) (end 154.94 82.55) (width 1.2192) (layer F.Cu) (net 5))
 (segment (start 152.305 79.915) (end 152.305 74.93) (width 1.2192) (layer F.Cu) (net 5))
 (segment (start 154.94 82.55) (end 152.305 79.915) (width 1.2192) (layer F.Cu) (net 5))
 (segment (start 98.425 96.52) (end 100.965 96.52) (width 1.2192) (layer B.Cu) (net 5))
 (segment (start 100.965 96.52) (end 103.505 96.52) (width 1.2192) (layer B.Cu) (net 5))
 (segment (start 103.505 96.52) (end 106.045 96.52) (width 1.2192) (layer B.Cu) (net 5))
 (segment (start 106.045 96.52) (end 108.585 96.52) (width 1.2192) (layer B.Cu) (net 5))
 (segment (start 108.585 96.52) (end 111.125 96.52) (width 1.2192) (layer B.Cu) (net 5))
 (segment (start 111.125 96.52) (end 113.665 96.52) (width 1.2192) (layer B.Cu) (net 5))
 (segment (start 113.665 96.52) (end 116.205 96.52) (width 1.2192) (layer B.Cu) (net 5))
 (segment (start 116.205 96.52) (end 118.745 96.52) (width 1.2192) (layer B.Cu) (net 5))
 (segment (start 118.745 96.52) (end 121.285 96.52) (width 1.2192) (layer B.Cu) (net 5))
 (segment (start 121.285 96.52) (end 123.825 96.52) (width 1.2192) (layer B.Cu) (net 5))
 (segment (start 123.825 96.52) (end 126.365 96.52) (width 1.2192) (layer B.Cu) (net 5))
 (segment (start 126.365 96.52) (end 128.905 96.52) (width 1.2192) (layer B.Cu) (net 5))
 (segment (start 128.905 96.52) (end 131.445 96.52) (width 1.2192) (layer B.Cu) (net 5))
 (segment (start 131.445 96.52) (end 133.985 96.52) (width 1.2192) (layer B.Cu) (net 5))
 (segment (start 133.985 96.52) (end 136.525 96.52) (width 1.2192) (layer B.Cu) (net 5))
 (segment (start 136.525 96.52) (end 138.43 96.52) (width 1.2192) (layer B.Cu) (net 5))
 (segment (start 138.43 96.52) (end 139.7 97.79) (width 1.2192) (layer B.Cu) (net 5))
 (segment (start 139.7 97.79) (end 142.875 97.79) (width 1.2192) (layer B.Cu) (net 5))
 (segment (start 142.875 97.79) (end 144.78 95.885) (width 1.2192) (layer B.Cu) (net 5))
 (segment (start 144.78 95.885) (end 144.78 94.3356) (width 1.2192) (layer B.Cu) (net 5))
 (segment (start 146.304 93.0656) (end 146.05 93.0656) (width 1.2192) (layer B.Cu) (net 5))
 (segment (start 147.32 94.0816) (end 146.304 93.0656) (width 1.2192) (layer B.Cu) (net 5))
 (segment (start 147.32 95.25) (end 147.32 94.0816) (width 1.2192) (layer B.Cu) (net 5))
 (segment (start 144.78 94.3356) (end 146.05 93.0656) (width 1.2192) (layer B.Cu) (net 5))
 (segment (start 146.05 93.0656) (end 150.2156 88.9) (width 1.2192) (layer B.Cu) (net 5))
 (segment (start 90.805 106.68) (end 90.805 106.045) (width 0.8128) (layer B.Cu) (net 1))
 (segment (start 90.805 106.045) (end 93.345 103.505) (width 0.8128) (layer B.Cu) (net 1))
 (segment (start 93.345 103.505) (end 93.345 99.695) (width 0.8128) (layer B.Cu) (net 1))
 (segment (start 91.44 97.79) (end 91.44 94.365) (width 0.8128) (layer B.Cu) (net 1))
 (segment (start 93.345 99.695) (end 91.44 97.79) (width 0.8128) (layer B.Cu) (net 1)))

